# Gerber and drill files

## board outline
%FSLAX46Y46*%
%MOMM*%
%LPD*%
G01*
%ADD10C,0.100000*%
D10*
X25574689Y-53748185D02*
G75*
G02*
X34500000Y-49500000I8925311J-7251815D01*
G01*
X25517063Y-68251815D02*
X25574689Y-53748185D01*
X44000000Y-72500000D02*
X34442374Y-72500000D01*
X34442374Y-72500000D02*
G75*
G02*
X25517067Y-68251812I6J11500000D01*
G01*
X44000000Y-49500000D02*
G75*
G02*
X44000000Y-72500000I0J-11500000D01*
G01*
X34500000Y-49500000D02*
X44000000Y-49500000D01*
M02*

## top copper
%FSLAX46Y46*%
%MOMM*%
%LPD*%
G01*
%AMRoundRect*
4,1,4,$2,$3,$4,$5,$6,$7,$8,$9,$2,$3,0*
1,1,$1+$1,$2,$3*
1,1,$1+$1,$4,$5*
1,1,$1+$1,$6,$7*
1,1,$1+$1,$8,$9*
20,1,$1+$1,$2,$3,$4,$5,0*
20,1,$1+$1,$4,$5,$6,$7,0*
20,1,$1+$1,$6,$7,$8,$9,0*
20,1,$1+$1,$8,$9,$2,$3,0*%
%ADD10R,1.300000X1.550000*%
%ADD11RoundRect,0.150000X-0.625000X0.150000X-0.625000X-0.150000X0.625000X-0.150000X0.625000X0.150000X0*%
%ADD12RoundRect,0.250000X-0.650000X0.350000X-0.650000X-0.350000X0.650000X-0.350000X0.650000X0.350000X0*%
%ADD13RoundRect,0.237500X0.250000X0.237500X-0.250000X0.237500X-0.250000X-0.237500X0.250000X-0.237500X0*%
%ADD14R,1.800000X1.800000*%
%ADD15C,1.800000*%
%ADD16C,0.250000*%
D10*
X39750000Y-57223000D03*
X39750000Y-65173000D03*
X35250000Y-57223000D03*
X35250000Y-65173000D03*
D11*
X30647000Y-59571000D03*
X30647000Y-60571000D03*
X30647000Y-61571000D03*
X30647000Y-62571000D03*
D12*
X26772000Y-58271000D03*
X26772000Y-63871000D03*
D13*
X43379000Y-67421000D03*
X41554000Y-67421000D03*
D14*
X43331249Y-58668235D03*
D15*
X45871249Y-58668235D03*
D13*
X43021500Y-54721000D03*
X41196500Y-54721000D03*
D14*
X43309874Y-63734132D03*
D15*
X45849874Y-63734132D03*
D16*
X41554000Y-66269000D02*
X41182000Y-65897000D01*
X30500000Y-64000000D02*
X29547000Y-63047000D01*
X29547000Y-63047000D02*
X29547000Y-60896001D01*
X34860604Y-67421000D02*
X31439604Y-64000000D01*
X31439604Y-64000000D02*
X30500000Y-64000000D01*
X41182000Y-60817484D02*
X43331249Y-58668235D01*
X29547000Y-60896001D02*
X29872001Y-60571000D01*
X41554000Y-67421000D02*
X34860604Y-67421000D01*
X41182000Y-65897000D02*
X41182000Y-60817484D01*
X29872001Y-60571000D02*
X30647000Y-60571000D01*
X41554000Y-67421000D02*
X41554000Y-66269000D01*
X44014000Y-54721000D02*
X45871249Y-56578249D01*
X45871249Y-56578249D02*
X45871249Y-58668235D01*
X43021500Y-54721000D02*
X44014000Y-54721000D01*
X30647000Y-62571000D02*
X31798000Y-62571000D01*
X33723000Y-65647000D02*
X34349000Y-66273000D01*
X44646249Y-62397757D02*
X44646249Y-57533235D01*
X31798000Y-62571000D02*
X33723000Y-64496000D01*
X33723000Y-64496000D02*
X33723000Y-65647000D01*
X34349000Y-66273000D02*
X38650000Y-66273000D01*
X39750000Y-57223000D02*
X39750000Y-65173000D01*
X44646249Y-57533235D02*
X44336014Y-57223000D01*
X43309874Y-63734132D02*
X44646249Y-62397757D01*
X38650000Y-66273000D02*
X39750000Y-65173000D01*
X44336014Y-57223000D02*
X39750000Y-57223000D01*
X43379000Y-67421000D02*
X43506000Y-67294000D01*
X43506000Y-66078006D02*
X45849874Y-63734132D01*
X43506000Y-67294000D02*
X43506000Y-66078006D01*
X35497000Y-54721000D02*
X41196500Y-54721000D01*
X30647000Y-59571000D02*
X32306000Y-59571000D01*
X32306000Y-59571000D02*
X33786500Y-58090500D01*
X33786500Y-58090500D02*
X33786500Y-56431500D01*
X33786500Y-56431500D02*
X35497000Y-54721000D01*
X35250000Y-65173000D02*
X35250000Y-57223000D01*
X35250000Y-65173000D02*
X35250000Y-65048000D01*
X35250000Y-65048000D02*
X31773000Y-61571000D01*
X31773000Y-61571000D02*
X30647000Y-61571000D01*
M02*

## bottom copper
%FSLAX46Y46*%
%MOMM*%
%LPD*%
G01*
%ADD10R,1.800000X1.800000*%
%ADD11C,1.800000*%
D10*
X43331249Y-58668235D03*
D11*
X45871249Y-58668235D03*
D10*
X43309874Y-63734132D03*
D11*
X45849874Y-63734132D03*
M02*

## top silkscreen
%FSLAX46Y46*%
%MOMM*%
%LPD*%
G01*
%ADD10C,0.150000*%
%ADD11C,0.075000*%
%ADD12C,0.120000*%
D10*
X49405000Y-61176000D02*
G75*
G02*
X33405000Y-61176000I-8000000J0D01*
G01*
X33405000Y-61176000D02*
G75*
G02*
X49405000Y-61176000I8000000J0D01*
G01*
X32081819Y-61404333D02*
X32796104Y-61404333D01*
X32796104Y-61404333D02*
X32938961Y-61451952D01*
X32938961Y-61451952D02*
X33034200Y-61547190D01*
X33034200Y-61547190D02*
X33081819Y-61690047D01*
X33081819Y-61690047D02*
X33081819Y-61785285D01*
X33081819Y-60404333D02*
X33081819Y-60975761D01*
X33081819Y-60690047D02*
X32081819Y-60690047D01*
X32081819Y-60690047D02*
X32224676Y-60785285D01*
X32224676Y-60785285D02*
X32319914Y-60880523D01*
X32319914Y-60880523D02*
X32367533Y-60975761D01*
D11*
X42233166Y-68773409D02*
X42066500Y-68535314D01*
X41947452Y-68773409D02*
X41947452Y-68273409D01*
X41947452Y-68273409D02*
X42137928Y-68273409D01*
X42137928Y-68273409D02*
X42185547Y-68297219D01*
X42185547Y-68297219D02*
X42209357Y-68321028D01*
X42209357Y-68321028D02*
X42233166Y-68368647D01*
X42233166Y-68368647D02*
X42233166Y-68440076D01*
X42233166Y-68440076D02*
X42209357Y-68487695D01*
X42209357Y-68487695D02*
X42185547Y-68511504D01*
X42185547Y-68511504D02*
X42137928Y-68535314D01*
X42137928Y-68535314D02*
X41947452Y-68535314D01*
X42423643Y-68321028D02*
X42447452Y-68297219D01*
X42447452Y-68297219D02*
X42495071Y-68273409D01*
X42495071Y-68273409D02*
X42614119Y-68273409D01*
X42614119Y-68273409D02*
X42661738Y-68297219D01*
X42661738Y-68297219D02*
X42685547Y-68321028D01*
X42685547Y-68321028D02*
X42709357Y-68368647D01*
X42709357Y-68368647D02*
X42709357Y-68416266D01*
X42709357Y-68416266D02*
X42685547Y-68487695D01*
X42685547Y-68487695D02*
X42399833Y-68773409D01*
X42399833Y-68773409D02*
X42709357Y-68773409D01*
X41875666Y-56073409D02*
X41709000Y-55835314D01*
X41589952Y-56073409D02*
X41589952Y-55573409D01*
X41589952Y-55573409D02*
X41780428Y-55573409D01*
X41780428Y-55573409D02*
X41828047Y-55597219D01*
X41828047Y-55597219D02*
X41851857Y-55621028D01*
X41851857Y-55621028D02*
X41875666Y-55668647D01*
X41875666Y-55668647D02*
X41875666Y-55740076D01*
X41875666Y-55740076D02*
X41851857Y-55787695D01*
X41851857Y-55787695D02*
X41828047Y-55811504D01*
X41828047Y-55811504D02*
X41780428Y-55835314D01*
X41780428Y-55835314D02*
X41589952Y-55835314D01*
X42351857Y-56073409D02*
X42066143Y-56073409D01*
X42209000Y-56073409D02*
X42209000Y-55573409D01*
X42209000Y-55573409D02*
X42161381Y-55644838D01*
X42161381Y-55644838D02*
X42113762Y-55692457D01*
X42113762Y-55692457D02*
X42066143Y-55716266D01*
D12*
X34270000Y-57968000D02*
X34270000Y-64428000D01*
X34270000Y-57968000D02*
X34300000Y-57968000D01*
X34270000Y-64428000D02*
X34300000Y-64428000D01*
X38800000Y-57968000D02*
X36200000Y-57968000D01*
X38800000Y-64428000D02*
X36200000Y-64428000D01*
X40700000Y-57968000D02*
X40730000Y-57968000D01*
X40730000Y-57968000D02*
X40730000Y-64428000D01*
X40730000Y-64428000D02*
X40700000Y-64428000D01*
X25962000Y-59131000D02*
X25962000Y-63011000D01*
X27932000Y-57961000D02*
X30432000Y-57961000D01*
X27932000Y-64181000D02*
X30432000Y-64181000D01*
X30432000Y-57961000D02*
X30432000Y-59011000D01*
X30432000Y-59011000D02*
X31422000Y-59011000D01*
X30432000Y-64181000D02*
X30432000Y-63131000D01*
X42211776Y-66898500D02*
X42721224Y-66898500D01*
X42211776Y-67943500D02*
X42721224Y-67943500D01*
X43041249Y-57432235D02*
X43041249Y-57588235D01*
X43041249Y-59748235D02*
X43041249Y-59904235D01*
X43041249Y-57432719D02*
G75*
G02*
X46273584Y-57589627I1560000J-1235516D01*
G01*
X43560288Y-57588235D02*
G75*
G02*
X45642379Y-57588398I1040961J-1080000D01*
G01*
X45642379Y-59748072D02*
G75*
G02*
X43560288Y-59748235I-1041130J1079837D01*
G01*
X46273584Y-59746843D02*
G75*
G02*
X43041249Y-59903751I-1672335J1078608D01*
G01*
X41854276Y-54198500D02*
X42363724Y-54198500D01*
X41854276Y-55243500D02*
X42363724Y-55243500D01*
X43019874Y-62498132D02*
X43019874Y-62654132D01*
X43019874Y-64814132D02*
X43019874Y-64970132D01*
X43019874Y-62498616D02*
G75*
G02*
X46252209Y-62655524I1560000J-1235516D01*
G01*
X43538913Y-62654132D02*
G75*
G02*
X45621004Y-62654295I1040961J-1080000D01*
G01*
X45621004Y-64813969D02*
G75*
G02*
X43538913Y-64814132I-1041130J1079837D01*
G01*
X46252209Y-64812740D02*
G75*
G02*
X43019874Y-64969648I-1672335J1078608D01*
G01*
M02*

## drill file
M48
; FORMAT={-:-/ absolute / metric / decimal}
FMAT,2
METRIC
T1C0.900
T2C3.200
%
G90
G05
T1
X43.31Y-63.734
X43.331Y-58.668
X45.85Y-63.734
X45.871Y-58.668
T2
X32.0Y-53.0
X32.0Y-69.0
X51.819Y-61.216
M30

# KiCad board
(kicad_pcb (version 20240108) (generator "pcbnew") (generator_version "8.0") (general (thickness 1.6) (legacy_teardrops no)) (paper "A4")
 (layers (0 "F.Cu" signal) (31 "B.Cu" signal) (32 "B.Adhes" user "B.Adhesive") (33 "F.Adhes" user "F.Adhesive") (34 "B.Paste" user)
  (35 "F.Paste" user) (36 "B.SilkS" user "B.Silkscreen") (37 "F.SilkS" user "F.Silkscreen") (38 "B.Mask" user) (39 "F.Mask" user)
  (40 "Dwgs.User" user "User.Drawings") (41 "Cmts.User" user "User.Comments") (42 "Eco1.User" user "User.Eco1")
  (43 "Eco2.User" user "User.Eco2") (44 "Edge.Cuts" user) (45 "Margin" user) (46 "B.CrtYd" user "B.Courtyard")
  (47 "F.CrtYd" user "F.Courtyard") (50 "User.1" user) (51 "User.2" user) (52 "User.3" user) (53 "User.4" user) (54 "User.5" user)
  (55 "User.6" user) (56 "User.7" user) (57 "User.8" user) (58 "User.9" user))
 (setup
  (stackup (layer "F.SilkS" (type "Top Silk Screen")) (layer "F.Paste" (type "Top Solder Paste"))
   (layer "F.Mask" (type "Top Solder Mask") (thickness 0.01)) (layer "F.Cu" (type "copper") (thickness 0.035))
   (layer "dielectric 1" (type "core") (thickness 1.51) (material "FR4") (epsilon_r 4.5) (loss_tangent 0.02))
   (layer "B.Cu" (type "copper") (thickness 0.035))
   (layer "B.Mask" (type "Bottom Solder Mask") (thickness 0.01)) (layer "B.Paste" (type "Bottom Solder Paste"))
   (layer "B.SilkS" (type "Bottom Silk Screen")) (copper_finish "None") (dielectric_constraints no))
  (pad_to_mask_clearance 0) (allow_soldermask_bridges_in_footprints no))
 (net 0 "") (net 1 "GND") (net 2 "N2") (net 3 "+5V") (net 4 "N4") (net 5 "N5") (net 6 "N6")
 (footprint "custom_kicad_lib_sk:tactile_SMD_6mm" (layer "F.Cu") (at 37.5 61.198 -90)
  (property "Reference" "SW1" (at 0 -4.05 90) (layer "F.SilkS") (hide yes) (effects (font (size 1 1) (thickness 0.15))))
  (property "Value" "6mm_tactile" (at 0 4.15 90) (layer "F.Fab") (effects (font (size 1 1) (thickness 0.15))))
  (fp_line (start -3.23 3.23) (end 3.23 3.23) (stroke (width 0.12) (type solid)) (layer "F.SilkS"))
  (fp_line (start -3.23 3.23) (end -3.23 3.2) (stroke (width 0.12) (type solid)) (layer "F.SilkS"))
  (fp_line (start 3.23 3.23) (end 3.23 3.2) (stroke (width 0.12) (type solid)) (layer "F.SilkS"))
  (fp_line (start -3.23 -1.3) (end -3.23 1.3) (stroke (width 0.12) (type solid)) (layer "F.SilkS"))
  (fp_line (start 3.23 -1.3) (end 3.23 1.3) (stroke (width 0.12) (type solid)) (layer "F.SilkS"))
  (fp_line (start -3.23 -3.2) (end -3.23 -3.23) (stroke (width 0.12) (type solid)) (layer "F.SilkS"))
  (fp_line (start -3.23 -3.23) (end 3.23 -3.23) (stroke (width 0.12) (type solid)) (layer "F.SilkS"))
  (fp_line (start 3.23 -3.23) (end 3.23 -3.2) (stroke (width 0.12) (type solid)) (layer "F.SilkS"))
  (pad "1" smd rect (at -3.975 -2.25 270) (size 1.55 1.3) (layers "F.Cu" "F.Paste" "F.Mask") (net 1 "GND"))
  (pad "1" smd rect (at 3.975 -2.25 270) (size 1.55 1.3) (layers "F.Cu" "F.Paste" "F.Mask") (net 1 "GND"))
  (pad "2" smd rect (at -3.975 2.25 270) (size 1.55 1.3) (layers "F.Cu" "F.Paste" "F.Mask") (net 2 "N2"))
  (pad "2" smd rect (at 3.975 2.25 270) (size 1.55 1.3) (layers "F.Cu" "F.Paste" "F.Mask") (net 2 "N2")))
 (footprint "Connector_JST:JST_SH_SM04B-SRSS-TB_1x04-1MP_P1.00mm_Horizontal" (layer "F.Cu") (at 28.647 61.071 -90)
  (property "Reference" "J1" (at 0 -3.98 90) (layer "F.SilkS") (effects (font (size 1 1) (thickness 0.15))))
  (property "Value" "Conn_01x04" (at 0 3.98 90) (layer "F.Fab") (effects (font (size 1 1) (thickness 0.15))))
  (fp_line (start -1.94 2.685) (end 1.94 2.685) (stroke (width 0.12) (type solid)) (layer "F.SilkS"))
  (fp_line (start -3.11 0.715) (end -3.11 -1.785) (stroke (width 0.12) (type solid)) (layer "F.SilkS"))
  (fp_line (start 3.11 0.715) (end 3.11 -1.785) (stroke (width 0.12) (type solid)) (layer "F.SilkS"))
  (fp_line (start -3.11 -1.785) (end -2.06 -1.785) (stroke (width 0.12) (type solid)) (layer "F.SilkS"))
  (fp_line (start -2.06 -1.785) (end -2.06 -2.775) (stroke (width 0.12) (type solid)) (layer "F.SilkS"))
  (fp_line (start 3.11 -1.785) (end 2.06 -1.785) (stroke (width 0.12) (type solid)) (layer "F.SilkS"))
  (pad "1" smd roundrect (at -1.5 -2 270) (size 0.6 1.55) (layers "F.Cu" "F.Paste" "F.Mask") (roundrect_rratio 0.25) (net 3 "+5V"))
  (pad "2" smd roundrect (at -0.5 -2 270) (size 0.6 1.55) (layers "F.Cu" "F.Paste" "F.Mask") (roundrect_rratio 0.25) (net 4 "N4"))
  (pad "3" smd roundrect (at 0.5 -2 270) (size 0.6 1.55) (layers "F.Cu" "F.Paste" "F.Mask") (roundrect_rratio 0.25) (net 2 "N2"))
  (pad "4" smd roundrect (at 1.5 -2 270) (size 0.6 1.55) (layers "F.Cu" "F.Paste" "F.Mask") (roundrect_rratio 0.25) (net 1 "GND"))
  (pad "MP" smd roundrect (at -2.8 1.875 270) (size 1.2 1.8) (layers "F.Cu" "F.Paste" "F.Mask") (roundrect_rratio 0.208333))
  (pad "MP" smd roundrect (at 2.8 1.875 270) (size 1.2 1.8) (layers "F.Cu" "F.Paste" "F.Mask") (roundrect_rratio 0.208333)))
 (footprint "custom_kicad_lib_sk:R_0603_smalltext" (layer "F.Cu") (at 42.4665 67.421 180)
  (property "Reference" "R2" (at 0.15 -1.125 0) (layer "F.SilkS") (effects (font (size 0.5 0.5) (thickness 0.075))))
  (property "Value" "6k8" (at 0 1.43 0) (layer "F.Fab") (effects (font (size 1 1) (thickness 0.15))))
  (fp_line (start 0.254724 0.5225) (end -0.254724 0.5225) (stroke (width 0.12) (type solid)) (layer "F.SilkS"))
  (fp_line (start 0.254724 -0.5225) (end -0.254724 -0.5225) (stroke (width 0.12) (type solid)) (layer "F.SilkS"))
  (pad "1" smd roundrect (at -0.9125 0 180) (size 0.975 0.95) (layers "F.Cu" "F.Paste" "F.Mask") (roundrect_rratio 0.25) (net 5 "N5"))
  (pad "2" smd roundrect (at 0.9125 0 180) (size 0.975 0.95) (layers "F.Cu" "F.Paste" "F.Mask") (roundrect_rratio 0.25) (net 4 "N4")))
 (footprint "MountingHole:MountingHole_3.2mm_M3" (layer "F.Cu") (at 51.819 61.216)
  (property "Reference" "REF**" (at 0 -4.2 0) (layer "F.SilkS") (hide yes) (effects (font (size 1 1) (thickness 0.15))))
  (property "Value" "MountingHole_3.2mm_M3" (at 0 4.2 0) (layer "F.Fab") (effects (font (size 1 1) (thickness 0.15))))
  (pad "" np_thru_hole circle (at 0 0) (size 3.2 3.2) (drill 3.2) (layers "F&B.Cu" "*.Mask")))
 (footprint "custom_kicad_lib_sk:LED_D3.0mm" (layer "F.Cu") (at 43.331249 58.668235)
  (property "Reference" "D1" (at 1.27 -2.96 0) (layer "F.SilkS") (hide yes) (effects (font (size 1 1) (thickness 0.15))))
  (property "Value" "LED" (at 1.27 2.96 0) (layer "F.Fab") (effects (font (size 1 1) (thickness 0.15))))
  (fp_line (start -0.29 -1.236) (end -0.29 -1.08) (stroke (width 0.12) (type solid)) (layer "F.SilkS"))
  (fp_line (start -0.29 1.08) (end -0.29 1.236) (stroke (width 0.12) (type solid)) (layer "F.SilkS"))
  (fp_arc (start -0.29 -1.235516) (mid 1.366487 -1.987659) (end 2.942335 -1.078608) (stroke (width 0.12) (type solid)) (layer "F.SilkS"))
  (fp_arc (start 0.229039 -1.08) (mid 1.270117 -1.5) (end 2.31113 -1.079837) (stroke (width 0.12) (type solid)) (layer "F.SilkS"))
  (fp_arc (start 2.31113 1.079837) (mid 1.270117 1.5) (end 0.229039 1.08) (stroke (width 0.12) (type solid)) (layer "F.SilkS"))
  (fp_arc (start 2.942335 1.078608) (mid 1.366487 1.987659) (end -0.29 1.235516) (stroke (width 0.12) (type solid)) (layer "F.SilkS"))
  (pad "1" thru_hole rect (at 0 0) (size 1.8 1.8) (drill 0.9) (layers "*.Cu" "*.Mask") (remove_unused_layers no) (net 4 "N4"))
  (pad "2" thru_hole circle (at 2.54 0) (size 1.8 1.8) (drill 0.9) (layers "*.Cu" "*.Mask") (remove_unused_layers no) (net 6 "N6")))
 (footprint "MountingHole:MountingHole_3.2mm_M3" (layer "F.Cu") (at 32 53)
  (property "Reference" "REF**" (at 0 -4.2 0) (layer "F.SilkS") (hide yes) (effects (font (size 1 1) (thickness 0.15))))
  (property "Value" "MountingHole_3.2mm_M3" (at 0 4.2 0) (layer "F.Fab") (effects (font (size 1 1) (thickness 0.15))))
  (pad "" np_thru_hole circle (at 0 0) (size 3.2 3.2) (drill 3.2) (layers "F&B.Cu" "*.Mask")))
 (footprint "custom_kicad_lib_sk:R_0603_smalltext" (layer "F.Cu") (at 42.109 54.721 180)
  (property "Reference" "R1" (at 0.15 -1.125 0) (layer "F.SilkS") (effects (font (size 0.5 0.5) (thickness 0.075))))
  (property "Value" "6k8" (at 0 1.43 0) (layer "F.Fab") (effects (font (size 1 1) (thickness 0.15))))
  (fp_line (start 0.254724 0.5225) (end -0.254724 0.5225) (stroke (width 0.12) (type solid)) (layer "F.SilkS"))
  (fp_line (start 0.254724 -0.5225) (end -0.254724 -0.5225) (stroke (width 0.12) (type solid)) (layer "F.SilkS"))
  (pad "1" smd roundrect (at -0.9125 0 180) (size 0.975 0.95) (layers "F.Cu" "F.Paste" "F.Mask") (roundrect_rratio 0.25) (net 6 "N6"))
  (pad "2" smd roundrect (at 0.9125 0 180) (size 0.975 0.95) (layers "F.Cu" "F.Paste" "F.Mask") (roundrect_rratio 0.25) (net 3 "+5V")))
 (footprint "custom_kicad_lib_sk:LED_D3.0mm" (layer "F.Cu") (at 43.309874 63.734132)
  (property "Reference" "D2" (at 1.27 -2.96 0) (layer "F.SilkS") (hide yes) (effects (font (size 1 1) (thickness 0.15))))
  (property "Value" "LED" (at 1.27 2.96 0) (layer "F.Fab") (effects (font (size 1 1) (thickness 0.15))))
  (fp_line (start -0.29 -1.236) (end -0.29 -1.08) (stroke (width 0.12) (type solid)) (layer "F.SilkS"))
  (fp_line (start -0.29 1.08) (end -0.29 1.236) (stroke (width 0.12) (type solid)) (layer "F.SilkS"))
  (fp_arc (start -0.29 -1.235516) (mid 1.366487 -1.987659) (end 2.942335 -1.078608) (stroke (width 0.12) (type solid)) (layer "F.SilkS"))
  (fp_arc (start 0.229039 -1.08) (mid 1.270117 -1.5) (end 2.31113 -1.079837) (stroke (width 0.12) (type solid)) (layer "F.SilkS"))
  (fp_arc (start 2.31113 1.079837) (mid 1.270117 1.5) (end 0.229039 1.08) (stroke (width 0.12) (type solid)) (layer "F.SilkS"))
  (fp_arc (start 2.942335 1.078608) (mid 1.366487 1.987659) (end -0.29 1.235516) (stroke (width 0.12) (type solid)) (layer "F.SilkS"))
  (pad "1" thru_hole rect (at 0 0) (size 1.8 1.8) (drill 0.9) (layers "*.Cu" "*.Mask") (remove_unused_layers no) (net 1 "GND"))
  (pad "2" thru_hole circle (at 2.54 0) (size 1.8 1.8) (drill 0.9) (layers "*.Cu" "*.Mask") (remove_unused_layers no) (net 5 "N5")))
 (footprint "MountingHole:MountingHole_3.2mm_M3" (layer "F.Cu") (at 32 69)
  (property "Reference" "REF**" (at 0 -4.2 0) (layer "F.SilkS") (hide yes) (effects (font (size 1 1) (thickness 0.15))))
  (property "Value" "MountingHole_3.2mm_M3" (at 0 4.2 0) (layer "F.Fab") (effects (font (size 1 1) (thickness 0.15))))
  (pad "" np_thru_hole circle (at 0 0) (size 3.2 3.2) (drill 3.2) (layers "F&B.Cu" "*.Mask")))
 (gr_circle (center 41.405 61.176) (end 49.405 61.176) (stroke (width 0.15) (type default)) (fill none) (layer "F.SilkS"))
 (gr_arc (start 25.574689 53.748185) (mid 29.557626 50.616218) (end 34.5 49.5) (stroke (width 0.1) (type default)) (layer "Edge.Cuts"))
 (gr_line (start 25.517063 68.251815) (end 25.574689 53.748185) (stroke (width 0.1) (type default)) (layer "Edge.Cuts"))
 (gr_line (start 44 72.5) (end 34.442374 72.5) (stroke (width 0.1) (type default)) (layer "Edge.Cuts"))
 (gr_arc (start 34.442374 72.5) (mid 29.5 71.383782) (end 25.517063 68.251815) (stroke (width 0.1) (type default)) (layer "Edge.Cuts"))
 (gr_arc (start 44 49.5) (mid 55.5 61) (end 44 72.5) (stroke (width 0.1) (type default)) (layer "Edge.Cuts"))
 (gr_line (start 34.5 49.5) (end 44 49.5) (stroke (width 0.1) (type default)) (layer "Edge.Cuts"))
 (segment (start 41.554 66.269) (end 41.182 65.897) (width 0.25) (layer "F.Cu") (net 4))
 (segment (start 30.5 64) (end 29.547 63.047) (width 0.25) (layer "F.Cu") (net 4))
 (segment (start 29.547 63.047) (end 29.547 60.896001) (width 0.25) (layer "F.Cu") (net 4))
 (segment (start 34.860604 67.421) (end 31.439604 64) (width 0.25) (layer "F.Cu") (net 4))
 (segment (start 31.439604 64) (end 30.5 64) (width 0.25) (layer "F.Cu") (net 4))
 (segment (start 41.182 60.817484) (end 43.331249 58.668235) (width 0.25) (layer "F.Cu") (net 4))
 (segment (start 29.547 60.896001) (end 29.872001 60.571) (width 0.25) (layer "F.Cu") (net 4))
 (segment (start 41.554 67.421) (end 34.860604 67.421) (width 0.25) (layer "F.Cu") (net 4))
 (segment (start 41.182 65.897) (end 41.182 60.817484) (width 0.25) (layer "F.Cu") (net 4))
 (segment (start 29.872001 60.571) (end 30.647 60.571) (width 0.25) (layer "F.Cu") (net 4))
 (segment (start 41.554 67.421) (end 41.554 66.269) (width 0.25) (layer "F.Cu") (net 4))
 (segment (start 44.014 54.721) (end 45.871249 56.578249) (width 0.25) (layer "F.Cu") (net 6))
 (segment (start 45.871249 56.578249) (end 45.871249 58.668235) (width 0.25) (layer "F.Cu") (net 6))
 (segment (start 43.0215 54.721) (end 44.014 54.721) (width 0.25) (layer "F.Cu") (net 6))
 (segment (start 30.647 62.571) (end 31.798 62.571) (width 0.25) (layer "F.Cu") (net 1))
 (segment (start 33.723 65.647) (end 34.349 66.273) (width 0.25) (layer "F.Cu") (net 1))
 (segment (start 44.646249 62.397757) (end 44.646249 57.533235) (width 0.25) (layer "F.Cu") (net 1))
 (segment (start 31.798 62.571) (end 33.723 64.496) (width 0.25) (layer "F.Cu") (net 1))
 (segment (start 33.723 64.496) (end 33.723 65.647) (width 0.25) (layer "F.Cu") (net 1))
 (segment (start 34.349 66.273) (end 38.65 66.273) (width 0.25) (layer "F.Cu") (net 1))
 (segment (start 39.75 57.223) (end 39.75 65.173) (width 0.25) (layer "F.Cu") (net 1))
 (segment (start 44.646249 57.533235) (end 44.336014 57.223) (width 0.25) (layer "F.Cu") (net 1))
 (segment (start 43.309874 63.734132) (end 44.646249 62.397757) (width 0.25) (layer "F.Cu") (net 1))
 (segment (start 38.65 66.273) (end 39.75 65.173) (width 0.25) (layer "F.Cu") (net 1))
 (segment (start 44.336014 57.223) (end 39.75 57.223) (width 0.25) (layer "F.Cu") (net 1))
 (segment (start 43.379 67.421) (end 43.506 67.294) (width 0.25) (layer "F.Cu") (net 5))
 (segment (start 43.506 66.078006) (end 45.849874 63.734132) (width 0.25) (layer "F.Cu") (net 5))
 (segment (start 43.506 67.294) (end 43.506 66.078006) (width 0.25) (layer "F.Cu") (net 5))
 (segment (start 35.497 54.721) (end 41.1965 54.721) (width 0.25) (layer "F.Cu") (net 3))
 (segment (start 30.647 59.571) (end 32.306 59.571) (width 0.25) (layer "F.Cu") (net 3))
 (segment (start 32.306 59.571) (end 33.7865 58.0905) (width 0.25) (layer "F.Cu") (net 3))
 (segment (start 33.7865 58.0905) (end 33.7865 56.4315) (width 0.25) (layer "F.Cu") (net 3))
 (segment (start 33.7865 56.4315) (end 35.497 54.721) (width 0.25) (layer "F.Cu") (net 3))
 (segment (start 35.25 65.173) (end 35.25 57.223) (width 0.25) (layer "F.Cu") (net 2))
 (segment (start 35.25 65.173) (end 35.25 65.048) (width 0.25) (layer "F.Cu") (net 2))
 (segment (start 35.25 65.048) (end 31.773 61.571) (width 0.25) (layer "F.Cu") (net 2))
 (segment (start 31.773 61.571) (end 30.647 61.571) (width 0.25) (layer "F.Cu") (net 2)))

